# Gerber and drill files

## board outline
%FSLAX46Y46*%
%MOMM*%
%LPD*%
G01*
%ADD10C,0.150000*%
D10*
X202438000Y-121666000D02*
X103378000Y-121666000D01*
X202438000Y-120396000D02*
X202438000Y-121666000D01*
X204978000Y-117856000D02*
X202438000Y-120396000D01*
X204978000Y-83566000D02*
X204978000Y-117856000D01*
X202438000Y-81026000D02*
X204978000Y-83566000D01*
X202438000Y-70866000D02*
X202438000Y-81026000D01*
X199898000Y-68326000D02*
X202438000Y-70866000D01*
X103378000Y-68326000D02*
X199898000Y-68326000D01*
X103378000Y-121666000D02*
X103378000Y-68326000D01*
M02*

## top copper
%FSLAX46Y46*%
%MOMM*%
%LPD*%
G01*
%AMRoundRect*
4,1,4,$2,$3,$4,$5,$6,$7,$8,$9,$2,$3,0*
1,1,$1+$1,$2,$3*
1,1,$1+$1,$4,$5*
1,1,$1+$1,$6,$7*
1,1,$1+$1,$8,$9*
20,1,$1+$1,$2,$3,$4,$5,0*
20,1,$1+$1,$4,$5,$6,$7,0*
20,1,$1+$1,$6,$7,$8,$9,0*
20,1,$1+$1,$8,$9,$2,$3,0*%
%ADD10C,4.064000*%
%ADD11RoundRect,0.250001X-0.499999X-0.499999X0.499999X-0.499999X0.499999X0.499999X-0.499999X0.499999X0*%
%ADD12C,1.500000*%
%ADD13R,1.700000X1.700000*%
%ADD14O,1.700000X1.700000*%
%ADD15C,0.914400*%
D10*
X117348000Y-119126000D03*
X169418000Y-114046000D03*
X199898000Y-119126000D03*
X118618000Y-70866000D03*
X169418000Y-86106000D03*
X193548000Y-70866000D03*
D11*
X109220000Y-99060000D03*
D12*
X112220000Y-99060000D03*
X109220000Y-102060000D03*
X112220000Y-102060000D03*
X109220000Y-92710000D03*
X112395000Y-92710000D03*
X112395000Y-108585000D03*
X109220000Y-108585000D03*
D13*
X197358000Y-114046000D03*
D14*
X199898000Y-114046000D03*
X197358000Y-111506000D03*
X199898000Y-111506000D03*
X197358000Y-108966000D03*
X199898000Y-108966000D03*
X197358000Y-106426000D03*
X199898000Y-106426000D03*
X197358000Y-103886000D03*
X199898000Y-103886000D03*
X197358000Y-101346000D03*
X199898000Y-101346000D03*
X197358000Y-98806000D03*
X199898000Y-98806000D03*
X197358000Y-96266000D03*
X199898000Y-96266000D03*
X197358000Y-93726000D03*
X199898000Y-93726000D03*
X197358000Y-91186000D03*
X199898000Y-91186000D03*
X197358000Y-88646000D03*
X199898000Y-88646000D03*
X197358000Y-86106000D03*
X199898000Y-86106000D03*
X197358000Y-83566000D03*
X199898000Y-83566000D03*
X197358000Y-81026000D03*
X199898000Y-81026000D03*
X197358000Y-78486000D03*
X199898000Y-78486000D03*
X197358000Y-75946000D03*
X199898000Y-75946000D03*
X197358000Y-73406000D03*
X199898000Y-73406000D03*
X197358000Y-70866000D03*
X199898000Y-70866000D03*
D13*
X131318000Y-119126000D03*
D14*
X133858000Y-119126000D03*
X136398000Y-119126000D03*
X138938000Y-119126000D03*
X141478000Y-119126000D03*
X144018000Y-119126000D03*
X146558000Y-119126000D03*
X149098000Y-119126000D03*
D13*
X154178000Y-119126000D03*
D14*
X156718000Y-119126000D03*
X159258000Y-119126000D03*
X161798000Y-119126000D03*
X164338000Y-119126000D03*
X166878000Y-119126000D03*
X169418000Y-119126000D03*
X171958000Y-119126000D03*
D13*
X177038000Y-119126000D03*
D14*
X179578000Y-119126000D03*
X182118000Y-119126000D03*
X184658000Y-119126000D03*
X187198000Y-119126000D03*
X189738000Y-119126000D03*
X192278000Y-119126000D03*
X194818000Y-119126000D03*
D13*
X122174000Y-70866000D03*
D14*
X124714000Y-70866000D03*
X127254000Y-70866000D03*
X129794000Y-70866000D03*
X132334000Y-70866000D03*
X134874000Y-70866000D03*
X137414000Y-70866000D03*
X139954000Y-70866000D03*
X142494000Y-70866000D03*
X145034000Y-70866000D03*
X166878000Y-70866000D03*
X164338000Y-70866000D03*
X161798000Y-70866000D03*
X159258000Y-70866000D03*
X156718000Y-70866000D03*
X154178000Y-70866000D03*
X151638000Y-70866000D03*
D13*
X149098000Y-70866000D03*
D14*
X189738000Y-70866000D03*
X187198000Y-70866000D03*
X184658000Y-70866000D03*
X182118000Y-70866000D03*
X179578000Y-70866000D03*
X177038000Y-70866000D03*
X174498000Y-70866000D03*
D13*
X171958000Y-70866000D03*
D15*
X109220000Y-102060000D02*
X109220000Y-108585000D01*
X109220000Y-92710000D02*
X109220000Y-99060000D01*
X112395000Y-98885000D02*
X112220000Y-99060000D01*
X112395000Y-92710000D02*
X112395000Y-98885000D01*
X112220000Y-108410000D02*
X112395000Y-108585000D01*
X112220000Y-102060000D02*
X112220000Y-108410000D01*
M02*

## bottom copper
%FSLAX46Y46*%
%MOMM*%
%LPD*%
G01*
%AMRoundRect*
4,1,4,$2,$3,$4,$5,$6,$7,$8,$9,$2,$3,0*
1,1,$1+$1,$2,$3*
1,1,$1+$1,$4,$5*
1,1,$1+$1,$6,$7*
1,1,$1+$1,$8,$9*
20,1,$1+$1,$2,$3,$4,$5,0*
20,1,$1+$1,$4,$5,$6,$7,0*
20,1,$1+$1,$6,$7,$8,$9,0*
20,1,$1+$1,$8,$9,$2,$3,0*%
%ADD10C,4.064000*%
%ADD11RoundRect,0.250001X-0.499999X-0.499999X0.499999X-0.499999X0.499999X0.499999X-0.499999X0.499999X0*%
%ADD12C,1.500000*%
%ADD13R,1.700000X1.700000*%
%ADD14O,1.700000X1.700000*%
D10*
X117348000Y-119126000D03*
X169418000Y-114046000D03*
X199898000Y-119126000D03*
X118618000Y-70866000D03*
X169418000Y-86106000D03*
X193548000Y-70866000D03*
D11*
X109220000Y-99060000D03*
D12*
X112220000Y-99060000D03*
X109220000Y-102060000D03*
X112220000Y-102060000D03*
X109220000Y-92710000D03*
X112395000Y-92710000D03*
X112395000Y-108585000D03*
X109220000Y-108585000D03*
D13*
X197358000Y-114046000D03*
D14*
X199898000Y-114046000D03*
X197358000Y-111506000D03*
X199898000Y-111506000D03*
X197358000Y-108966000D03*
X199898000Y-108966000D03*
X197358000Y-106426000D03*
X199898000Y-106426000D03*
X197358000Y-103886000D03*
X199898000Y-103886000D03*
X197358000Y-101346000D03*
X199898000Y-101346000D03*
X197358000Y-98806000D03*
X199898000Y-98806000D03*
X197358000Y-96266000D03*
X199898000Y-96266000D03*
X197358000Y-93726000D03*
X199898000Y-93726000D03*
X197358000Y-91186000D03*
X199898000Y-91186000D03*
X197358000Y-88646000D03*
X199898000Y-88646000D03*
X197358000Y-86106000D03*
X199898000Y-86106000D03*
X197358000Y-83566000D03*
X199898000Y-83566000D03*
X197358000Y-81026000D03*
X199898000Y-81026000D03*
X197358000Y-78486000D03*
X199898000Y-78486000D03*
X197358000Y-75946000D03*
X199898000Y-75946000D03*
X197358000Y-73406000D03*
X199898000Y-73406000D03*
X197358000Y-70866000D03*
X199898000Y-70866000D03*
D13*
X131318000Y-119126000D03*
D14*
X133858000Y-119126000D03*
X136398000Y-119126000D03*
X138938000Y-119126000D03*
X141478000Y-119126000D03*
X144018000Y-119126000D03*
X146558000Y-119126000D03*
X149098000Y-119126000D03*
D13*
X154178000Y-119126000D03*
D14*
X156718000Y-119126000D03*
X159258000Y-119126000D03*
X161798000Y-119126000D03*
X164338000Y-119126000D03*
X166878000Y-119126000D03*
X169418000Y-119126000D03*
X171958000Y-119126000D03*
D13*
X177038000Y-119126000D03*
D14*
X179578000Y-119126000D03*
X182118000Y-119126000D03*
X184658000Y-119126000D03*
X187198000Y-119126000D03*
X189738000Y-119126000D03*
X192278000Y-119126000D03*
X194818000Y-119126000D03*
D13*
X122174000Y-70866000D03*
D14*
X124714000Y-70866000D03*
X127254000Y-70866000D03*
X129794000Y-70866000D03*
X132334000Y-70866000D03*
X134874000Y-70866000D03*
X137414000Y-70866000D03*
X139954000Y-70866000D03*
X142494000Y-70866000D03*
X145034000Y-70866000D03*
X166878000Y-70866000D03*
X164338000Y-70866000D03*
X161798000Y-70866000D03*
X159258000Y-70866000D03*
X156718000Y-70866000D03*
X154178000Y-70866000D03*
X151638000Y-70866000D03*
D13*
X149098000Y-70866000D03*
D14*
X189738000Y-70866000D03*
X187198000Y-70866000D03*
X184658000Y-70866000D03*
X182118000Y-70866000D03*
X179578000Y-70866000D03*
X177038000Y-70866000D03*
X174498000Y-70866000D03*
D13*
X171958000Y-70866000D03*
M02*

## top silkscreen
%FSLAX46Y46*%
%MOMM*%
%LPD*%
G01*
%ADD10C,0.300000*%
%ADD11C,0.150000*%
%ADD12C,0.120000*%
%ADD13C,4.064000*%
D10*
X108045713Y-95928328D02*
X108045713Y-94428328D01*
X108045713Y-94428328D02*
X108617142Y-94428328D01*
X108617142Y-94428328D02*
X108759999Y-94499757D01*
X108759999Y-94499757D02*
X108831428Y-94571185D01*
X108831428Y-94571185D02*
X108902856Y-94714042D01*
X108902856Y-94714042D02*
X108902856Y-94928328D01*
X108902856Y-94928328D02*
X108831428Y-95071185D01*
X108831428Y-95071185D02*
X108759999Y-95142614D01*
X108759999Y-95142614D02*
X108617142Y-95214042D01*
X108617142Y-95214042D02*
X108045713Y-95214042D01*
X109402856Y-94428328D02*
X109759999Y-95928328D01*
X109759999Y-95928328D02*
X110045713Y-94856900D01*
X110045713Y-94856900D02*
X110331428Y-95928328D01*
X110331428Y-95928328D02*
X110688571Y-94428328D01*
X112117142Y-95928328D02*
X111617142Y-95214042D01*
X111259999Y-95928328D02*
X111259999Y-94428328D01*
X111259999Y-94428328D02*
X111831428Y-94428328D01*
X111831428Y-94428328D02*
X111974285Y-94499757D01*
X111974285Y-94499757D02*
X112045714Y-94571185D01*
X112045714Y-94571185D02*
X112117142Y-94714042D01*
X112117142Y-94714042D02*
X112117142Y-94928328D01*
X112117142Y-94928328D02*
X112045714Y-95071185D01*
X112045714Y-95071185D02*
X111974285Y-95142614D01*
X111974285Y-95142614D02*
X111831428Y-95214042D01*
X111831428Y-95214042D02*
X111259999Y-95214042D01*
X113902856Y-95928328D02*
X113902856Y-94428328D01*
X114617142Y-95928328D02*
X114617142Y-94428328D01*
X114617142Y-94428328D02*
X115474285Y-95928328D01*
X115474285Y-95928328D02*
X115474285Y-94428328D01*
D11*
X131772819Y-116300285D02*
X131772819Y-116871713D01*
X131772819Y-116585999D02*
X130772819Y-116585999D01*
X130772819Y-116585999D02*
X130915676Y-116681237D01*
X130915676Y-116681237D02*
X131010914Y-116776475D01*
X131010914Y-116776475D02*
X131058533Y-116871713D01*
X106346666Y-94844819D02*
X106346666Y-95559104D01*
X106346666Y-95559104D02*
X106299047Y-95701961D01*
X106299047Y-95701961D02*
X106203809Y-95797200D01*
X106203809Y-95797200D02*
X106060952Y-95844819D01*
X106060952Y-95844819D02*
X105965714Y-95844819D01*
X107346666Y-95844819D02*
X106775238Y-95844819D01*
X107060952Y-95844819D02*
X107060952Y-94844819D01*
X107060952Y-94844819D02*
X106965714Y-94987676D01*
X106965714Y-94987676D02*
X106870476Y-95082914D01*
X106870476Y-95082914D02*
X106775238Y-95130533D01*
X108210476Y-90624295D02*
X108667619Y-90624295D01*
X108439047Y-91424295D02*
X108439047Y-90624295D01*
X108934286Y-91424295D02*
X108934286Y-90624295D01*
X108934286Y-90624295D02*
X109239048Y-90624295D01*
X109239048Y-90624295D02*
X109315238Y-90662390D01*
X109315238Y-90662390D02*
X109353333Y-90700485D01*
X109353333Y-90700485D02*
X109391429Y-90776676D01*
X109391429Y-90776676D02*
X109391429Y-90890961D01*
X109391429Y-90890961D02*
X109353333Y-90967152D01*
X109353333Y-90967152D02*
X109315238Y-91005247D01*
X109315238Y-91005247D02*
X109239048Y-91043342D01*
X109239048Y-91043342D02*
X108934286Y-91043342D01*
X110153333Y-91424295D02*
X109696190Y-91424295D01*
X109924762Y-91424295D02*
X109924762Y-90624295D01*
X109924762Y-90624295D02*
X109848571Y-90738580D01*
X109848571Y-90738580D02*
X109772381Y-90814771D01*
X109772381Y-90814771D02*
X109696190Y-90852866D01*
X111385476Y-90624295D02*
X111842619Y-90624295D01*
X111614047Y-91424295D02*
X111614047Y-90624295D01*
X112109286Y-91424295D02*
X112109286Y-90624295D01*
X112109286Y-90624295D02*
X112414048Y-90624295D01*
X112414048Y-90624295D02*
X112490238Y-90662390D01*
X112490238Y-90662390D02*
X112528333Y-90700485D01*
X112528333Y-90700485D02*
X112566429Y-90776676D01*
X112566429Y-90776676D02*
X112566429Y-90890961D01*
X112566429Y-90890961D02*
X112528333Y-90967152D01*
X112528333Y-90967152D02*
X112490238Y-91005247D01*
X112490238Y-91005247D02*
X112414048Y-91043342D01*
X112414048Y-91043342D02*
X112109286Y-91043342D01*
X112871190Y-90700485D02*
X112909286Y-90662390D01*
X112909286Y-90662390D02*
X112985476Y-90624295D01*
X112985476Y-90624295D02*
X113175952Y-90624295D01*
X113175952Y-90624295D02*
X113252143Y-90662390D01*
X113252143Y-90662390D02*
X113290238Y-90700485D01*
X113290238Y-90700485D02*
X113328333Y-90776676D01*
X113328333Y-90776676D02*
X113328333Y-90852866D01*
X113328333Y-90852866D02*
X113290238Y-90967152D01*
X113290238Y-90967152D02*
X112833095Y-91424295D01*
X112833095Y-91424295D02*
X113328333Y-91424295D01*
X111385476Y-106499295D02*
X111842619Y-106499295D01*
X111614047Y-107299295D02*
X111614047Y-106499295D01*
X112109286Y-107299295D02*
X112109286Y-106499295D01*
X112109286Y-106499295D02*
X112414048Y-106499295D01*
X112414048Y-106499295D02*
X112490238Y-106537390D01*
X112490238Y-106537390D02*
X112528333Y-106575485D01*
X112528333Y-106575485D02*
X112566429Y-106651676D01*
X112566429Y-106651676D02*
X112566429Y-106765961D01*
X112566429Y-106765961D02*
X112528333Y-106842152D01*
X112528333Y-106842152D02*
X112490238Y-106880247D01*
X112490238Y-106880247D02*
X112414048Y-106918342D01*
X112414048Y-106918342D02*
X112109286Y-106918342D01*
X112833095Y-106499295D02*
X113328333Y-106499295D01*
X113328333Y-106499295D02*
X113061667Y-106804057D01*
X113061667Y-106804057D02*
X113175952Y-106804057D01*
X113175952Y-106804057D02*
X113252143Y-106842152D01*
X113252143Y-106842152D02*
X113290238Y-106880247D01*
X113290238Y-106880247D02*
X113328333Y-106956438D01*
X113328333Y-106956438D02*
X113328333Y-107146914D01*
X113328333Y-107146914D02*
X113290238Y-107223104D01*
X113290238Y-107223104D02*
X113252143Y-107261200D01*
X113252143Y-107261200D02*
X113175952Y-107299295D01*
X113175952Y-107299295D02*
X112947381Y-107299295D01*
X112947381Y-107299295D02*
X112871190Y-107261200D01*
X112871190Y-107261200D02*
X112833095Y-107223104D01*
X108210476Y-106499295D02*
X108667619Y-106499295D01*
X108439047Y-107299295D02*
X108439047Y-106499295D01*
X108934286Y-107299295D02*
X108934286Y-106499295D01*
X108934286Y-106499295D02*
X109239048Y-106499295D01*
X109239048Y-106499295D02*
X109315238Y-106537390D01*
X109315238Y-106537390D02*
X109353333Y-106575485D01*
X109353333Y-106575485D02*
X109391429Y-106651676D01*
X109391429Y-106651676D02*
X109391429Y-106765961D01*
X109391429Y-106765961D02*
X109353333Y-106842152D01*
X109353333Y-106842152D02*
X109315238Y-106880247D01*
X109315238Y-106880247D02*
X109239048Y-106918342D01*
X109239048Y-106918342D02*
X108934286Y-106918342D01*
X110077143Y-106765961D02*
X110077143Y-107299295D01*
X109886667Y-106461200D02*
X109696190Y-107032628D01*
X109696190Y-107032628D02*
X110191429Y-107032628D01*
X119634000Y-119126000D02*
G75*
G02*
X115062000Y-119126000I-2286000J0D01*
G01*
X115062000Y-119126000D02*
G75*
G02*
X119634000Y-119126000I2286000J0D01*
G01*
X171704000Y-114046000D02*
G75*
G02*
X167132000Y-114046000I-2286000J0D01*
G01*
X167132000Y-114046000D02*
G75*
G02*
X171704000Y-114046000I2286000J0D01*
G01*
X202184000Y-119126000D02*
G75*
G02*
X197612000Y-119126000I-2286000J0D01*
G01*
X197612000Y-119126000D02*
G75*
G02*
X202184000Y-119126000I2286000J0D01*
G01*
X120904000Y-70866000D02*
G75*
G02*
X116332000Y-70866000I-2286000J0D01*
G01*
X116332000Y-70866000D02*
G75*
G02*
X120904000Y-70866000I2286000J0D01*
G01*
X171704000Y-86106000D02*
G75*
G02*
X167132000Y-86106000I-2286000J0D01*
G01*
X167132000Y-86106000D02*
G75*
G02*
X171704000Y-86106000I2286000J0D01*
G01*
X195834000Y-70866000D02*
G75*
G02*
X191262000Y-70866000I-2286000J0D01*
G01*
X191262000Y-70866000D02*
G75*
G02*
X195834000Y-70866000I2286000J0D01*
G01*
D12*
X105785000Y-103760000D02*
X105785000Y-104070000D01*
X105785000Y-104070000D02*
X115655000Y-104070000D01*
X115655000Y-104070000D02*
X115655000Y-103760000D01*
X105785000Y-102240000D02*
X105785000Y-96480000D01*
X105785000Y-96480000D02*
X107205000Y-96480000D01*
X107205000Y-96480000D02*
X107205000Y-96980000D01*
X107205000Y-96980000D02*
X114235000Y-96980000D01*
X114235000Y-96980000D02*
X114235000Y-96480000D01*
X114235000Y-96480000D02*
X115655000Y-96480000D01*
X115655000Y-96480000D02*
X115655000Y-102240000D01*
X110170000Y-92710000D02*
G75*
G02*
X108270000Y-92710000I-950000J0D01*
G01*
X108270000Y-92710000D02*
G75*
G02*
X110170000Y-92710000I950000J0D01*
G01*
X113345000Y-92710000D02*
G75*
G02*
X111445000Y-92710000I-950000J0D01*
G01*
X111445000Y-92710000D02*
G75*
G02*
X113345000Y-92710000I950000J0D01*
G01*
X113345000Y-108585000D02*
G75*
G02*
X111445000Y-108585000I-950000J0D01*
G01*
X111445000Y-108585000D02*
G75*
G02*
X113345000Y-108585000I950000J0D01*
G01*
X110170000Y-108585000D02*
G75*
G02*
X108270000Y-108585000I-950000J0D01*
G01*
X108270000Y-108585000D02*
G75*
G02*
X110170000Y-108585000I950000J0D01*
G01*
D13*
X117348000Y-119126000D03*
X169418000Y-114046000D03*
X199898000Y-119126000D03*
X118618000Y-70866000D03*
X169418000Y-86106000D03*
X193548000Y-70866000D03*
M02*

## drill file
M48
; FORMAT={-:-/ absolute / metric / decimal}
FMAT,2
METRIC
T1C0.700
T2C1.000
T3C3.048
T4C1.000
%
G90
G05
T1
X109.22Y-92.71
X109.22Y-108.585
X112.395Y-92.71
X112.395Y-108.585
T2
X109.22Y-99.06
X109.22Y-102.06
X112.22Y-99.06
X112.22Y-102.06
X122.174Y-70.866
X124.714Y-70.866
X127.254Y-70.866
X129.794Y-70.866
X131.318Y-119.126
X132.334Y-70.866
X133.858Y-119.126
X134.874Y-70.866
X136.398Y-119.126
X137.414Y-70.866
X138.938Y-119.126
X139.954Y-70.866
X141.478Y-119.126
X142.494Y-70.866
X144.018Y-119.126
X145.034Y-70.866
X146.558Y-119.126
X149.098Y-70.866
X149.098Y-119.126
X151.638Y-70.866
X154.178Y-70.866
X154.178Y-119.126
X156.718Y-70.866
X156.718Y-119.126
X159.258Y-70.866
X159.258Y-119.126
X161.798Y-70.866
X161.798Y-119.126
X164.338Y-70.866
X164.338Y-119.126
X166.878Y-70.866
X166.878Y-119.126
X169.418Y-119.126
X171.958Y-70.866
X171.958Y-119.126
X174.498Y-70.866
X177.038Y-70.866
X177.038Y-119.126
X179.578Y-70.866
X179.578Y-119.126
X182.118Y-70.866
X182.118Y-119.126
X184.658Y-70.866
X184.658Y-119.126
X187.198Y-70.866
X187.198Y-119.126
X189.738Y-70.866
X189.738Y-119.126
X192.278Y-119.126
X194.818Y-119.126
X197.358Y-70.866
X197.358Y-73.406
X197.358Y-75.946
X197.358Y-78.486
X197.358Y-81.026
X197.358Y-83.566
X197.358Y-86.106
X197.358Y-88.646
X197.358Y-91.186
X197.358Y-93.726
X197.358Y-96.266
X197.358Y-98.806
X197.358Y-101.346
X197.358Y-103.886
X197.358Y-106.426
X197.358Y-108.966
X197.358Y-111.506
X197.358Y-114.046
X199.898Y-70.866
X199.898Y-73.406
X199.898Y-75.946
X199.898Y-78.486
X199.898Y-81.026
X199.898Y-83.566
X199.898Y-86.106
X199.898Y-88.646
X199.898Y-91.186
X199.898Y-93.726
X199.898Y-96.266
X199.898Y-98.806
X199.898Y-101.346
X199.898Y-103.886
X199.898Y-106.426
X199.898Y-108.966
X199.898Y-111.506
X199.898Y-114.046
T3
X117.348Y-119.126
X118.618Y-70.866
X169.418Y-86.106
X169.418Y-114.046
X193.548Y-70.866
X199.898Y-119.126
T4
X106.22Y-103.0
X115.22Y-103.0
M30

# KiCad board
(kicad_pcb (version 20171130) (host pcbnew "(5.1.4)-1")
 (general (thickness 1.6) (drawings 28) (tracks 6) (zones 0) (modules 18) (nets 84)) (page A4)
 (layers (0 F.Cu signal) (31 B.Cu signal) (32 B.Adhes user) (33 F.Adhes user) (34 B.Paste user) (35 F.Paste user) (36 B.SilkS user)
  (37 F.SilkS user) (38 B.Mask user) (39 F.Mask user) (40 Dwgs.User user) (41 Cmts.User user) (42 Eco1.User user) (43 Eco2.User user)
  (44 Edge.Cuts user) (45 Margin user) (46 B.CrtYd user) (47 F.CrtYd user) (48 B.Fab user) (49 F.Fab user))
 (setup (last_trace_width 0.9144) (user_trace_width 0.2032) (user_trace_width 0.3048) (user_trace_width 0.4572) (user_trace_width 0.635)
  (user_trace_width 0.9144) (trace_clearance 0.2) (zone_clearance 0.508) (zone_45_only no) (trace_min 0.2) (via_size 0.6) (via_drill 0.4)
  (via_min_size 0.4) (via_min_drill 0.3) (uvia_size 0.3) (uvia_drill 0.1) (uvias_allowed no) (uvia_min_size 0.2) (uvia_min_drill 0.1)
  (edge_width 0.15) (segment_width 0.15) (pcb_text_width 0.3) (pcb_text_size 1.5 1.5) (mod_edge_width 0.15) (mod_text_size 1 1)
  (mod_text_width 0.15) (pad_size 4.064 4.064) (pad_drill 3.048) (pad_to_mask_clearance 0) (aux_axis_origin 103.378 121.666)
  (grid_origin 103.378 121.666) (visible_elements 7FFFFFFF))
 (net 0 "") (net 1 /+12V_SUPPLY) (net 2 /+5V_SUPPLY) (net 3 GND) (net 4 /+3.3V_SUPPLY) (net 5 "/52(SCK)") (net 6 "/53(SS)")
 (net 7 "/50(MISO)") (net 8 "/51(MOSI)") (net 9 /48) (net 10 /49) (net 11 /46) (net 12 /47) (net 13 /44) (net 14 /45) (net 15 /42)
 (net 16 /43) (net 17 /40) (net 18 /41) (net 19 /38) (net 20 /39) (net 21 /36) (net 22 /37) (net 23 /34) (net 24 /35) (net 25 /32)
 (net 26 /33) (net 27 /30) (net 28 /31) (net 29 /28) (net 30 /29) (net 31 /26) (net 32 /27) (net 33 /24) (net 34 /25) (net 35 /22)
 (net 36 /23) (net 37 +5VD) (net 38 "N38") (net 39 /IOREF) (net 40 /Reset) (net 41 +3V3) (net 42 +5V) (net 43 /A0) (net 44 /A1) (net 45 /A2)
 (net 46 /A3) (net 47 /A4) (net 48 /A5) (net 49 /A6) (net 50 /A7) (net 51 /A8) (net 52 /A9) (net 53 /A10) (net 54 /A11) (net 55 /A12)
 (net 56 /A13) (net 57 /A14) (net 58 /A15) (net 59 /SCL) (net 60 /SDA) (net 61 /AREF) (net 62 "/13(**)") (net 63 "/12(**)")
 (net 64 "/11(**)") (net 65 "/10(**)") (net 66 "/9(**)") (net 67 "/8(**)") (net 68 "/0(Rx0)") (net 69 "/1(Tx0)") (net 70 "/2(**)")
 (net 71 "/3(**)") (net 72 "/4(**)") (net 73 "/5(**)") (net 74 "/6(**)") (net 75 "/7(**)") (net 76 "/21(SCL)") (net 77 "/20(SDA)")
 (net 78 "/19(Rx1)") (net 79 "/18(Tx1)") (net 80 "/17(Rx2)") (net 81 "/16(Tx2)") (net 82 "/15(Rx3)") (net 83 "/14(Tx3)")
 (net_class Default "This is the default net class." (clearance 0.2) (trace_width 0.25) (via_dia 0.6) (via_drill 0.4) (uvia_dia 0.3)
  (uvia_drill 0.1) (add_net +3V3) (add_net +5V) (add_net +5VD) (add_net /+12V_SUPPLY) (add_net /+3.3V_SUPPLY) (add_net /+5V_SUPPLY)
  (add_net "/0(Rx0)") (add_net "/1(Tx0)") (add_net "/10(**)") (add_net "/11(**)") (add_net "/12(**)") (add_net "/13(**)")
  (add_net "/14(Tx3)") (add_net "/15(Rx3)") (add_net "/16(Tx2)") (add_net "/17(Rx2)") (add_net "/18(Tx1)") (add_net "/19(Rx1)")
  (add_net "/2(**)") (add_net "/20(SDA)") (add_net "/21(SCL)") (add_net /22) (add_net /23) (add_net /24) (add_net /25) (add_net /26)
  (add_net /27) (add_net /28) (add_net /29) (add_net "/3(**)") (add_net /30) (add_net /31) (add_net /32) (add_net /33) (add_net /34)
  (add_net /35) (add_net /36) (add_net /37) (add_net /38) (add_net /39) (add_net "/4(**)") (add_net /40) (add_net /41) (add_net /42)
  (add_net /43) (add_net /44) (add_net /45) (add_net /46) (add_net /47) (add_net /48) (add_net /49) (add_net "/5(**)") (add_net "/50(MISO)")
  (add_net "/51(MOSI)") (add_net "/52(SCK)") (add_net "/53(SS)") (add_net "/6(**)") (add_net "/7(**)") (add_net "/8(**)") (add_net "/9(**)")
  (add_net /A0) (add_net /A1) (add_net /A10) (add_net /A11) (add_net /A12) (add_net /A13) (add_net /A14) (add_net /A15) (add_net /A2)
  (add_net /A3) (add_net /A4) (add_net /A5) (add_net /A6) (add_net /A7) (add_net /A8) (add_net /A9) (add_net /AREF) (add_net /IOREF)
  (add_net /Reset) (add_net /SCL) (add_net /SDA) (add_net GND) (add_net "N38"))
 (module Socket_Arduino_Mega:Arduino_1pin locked (layer F.Cu) (at 117.348 119.126)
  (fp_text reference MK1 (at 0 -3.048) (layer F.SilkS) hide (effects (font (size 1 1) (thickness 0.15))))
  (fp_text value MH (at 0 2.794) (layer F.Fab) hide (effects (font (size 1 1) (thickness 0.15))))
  (fp_circle (center 0 0) (end 0 -2.286) (layer F.SilkS) (width 0.15))
  (pad 1 thru_hole circle (at 0 0) (size 4.064 4.064) (drill 3.048) (layers *.Cu *.Mask F.SilkS)))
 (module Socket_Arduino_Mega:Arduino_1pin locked (layer F.Cu) (at 169.418 114.046)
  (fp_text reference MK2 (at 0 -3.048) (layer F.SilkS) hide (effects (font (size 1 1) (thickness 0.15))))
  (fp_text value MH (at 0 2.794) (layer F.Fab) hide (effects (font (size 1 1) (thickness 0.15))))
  (fp_circle (center 0 0) (end 0 -2.286) (layer F.SilkS) (width 0.15))
  (pad 1 thru_hole circle (at 0 0) (size 4.064 4.064) (drill 3.048) (layers *.Cu *.Mask F.SilkS)))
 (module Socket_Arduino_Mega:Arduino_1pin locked (layer F.Cu) (at 199.898 119.126)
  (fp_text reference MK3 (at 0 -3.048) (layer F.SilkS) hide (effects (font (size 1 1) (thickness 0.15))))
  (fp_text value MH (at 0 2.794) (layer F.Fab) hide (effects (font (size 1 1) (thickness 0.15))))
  (fp_circle (center 0 0) (end 0 -2.286) (layer F.SilkS) (width 0.15))
  (pad 1 thru_hole circle (at 0 0) (size 4.064 4.064) (drill 3.048) (layers *.Cu *.Mask F.SilkS)))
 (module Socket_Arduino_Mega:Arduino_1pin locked (layer F.Cu) (at 118.618 70.866)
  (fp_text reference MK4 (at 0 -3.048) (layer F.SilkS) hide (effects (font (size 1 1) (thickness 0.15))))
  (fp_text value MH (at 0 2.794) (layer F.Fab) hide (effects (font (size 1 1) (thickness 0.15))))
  (fp_circle (center 0 0) (end 0 -2.286) (layer F.SilkS) (width 0.15))
  (pad 1 thru_hole circle (at 0 0) (size 4.064 4.064) (drill 3.048) (layers *.Cu *.Mask F.SilkS)))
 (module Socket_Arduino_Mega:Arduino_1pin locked (layer F.Cu) (at 169.418 86.106)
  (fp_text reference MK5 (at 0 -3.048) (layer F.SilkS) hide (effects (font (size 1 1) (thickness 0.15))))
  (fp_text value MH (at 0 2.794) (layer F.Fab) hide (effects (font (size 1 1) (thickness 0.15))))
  (fp_circle (center 0 0) (end 0 -2.286) (layer F.SilkS) (width 0.15))
  (pad 1 thru_hole circle (at 0 0) (size 4.064 4.064) (drill 3.048) (layers *.Cu *.Mask F.SilkS)))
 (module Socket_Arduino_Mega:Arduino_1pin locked (layer F.Cu) (at 193.548 70.866)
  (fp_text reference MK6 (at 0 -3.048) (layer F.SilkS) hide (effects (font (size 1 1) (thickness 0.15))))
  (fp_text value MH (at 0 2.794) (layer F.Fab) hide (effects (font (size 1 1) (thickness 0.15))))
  (fp_circle (center 0 0) (end 0 -2.286) (layer F.SilkS) (width 0.15))
  (pad 1 thru_hole circle (at 0 0) (size 4.064 4.064) (drill 3.048) (layers *.Cu *.Mask F.SilkS)))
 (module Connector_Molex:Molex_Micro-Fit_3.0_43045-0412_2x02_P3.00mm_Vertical (layer F.Cu) (at 109.22 99.06)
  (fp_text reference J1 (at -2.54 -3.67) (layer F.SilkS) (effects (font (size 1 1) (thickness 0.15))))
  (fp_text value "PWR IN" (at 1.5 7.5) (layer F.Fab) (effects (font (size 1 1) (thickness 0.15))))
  (fp_line (start -3.435 4.7) (end -3.435 5.01) (layer F.SilkS) (width 0.12))
  (fp_line (start -3.435 5.01) (end 6.435 5.01) (layer F.SilkS) (width 0.12))
  (fp_line (start 6.435 5.01) (end 6.435 4.7) (layer F.SilkS) (width 0.12))
  (fp_line (start -3.435 3.18) (end -3.435 -2.58) (layer F.SilkS) (width 0.12))
  (fp_line (start -3.435 -2.58) (end -2.015 -2.58) (layer F.SilkS) (width 0.12))
  (fp_line (start -2.015 -2.58) (end -2.015 -2.08) (layer F.SilkS) (width 0.12))
  (fp_line (start -2.015 -2.08) (end 5.015 -2.08) (layer F.SilkS) (width 0.12))
  (fp_line (start 5.015 -2.08) (end 5.015 -2.58) (layer F.SilkS) (width 0.12))
  (fp_line (start 5.015 -2.58) (end 6.435 -2.58) (layer F.SilkS) (width 0.12))
  (fp_line (start 6.435 -2.58) (end 6.435 3.18) (layer F.SilkS) (width 0.12))
  (pad "" np_thru_hole circle (at -3 3.94) (size 1 1) (drill 1) (layers *.Cu *.Mask))
  (pad "" np_thru_hole circle (at 6 3.94) (size 1 1) (drill 1) (layers *.Cu *.Mask))
  (pad 1 thru_hole roundrect (at 0 0) (size 1.5 1.5) (drill 1) (layers *.Cu *.Mask) (roundrect_rratio 0.166667) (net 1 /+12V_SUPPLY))
  (pad 2 thru_hole circle (at 3 0) (size 1.5 1.5) (drill 1) (layers *.Cu *.Mask) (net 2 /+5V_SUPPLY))
  (pad 3 thru_hole circle (at 0 3) (size 1.5 1.5) (drill 1) (layers *.Cu *.Mask) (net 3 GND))
  (pad 4 thru_hole circle (at 3 3) (size 1.5 1.5) (drill 1) (layers *.Cu *.Mask) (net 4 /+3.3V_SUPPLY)))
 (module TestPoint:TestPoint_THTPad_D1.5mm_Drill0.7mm (layer F.Cu) (at 109.22 92.71)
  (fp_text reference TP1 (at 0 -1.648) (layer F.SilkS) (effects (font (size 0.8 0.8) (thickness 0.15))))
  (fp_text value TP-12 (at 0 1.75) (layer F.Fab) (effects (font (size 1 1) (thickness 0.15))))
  (fp_circle (center 0 0) (end 0 0.95) (layer F.SilkS) (width 0.12))
  (pad 1 thru_hole circle (at 0 0) (size 1.5 1.5) (drill 0.7) (layers *.Cu *.Mask) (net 1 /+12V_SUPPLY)))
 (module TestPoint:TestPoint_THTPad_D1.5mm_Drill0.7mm (layer F.Cu) (at 112.395 92.71)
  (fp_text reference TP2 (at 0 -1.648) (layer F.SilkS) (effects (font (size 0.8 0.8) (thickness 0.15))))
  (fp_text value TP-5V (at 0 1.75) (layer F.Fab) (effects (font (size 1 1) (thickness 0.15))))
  (fp_circle (center 0 0) (end 0 0.95) (layer F.SilkS) (width 0.12))
  (pad 1 thru_hole circle (at 0 0) (size 1.5 1.5) (drill 0.7) (layers *.Cu *.Mask) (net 2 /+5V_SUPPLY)))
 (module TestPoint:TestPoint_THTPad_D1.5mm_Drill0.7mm (layer F.Cu) (at 112.395 108.585)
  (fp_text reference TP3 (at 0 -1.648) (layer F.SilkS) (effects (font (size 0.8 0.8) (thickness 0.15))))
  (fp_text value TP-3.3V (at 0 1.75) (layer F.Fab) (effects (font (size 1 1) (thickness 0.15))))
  (fp_circle (center 0 0) (end 0 0.95) (layer F.SilkS) (width 0.12))
  (pad 1 thru_hole circle (at 0 0) (size 1.5 1.5) (drill 0.7) (layers *.Cu *.Mask) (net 4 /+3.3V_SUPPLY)))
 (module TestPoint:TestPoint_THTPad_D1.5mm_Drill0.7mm (layer F.Cu) (at 109.22 108.585)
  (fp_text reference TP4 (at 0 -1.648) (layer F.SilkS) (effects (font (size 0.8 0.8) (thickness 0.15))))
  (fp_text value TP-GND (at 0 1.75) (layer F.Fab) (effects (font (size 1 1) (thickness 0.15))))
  (fp_circle (center 0 0) (end 0 0.95) (layer F.SilkS) (width 0.12))
  (pad 1 thru_hole circle (at 0 0) (size 1.5 1.5) (drill 0.7) (layers *.Cu *.Mask) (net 3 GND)))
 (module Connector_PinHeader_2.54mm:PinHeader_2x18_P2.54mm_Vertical (layer B.Cu) (at 197.358 114.046)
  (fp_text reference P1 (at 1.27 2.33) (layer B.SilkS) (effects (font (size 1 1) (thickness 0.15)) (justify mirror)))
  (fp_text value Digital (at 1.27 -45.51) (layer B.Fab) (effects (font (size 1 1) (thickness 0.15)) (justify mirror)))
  (pad 1 thru_hole rect (at 0 0) (size 1.7 1.7) (drill 1) (layers *.Cu *.Mask) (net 3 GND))
  (pad 2 thru_hole oval (at 2.54 0) (size 1.7 1.7) (drill 1) (layers *.Cu *.Mask) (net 3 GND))
  (pad 3 thru_hole oval (at 0 -2.54) (size 1.7 1.7) (drill 1) (layers *.Cu *.Mask) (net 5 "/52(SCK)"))
  (pad 4 thru_hole oval (at 2.54 -2.54) (size 1.7 1.7) (drill 1) (layers *.Cu *.Mask) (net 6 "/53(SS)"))
  (pad 5 thru_hole oval (at 0 -5.08) (size 1.7 1.7) (drill 1) (layers *.Cu *.Mask) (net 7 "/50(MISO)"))
  (pad 6 thru_hole oval (at 2.54 -5.08) (size 1.7 1.7) (drill 1) (layers *.Cu *.Mask) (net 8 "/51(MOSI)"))
  (pad 7 thru_hole oval (at 0 -7.62) (size 1.7 1.7) (drill 1) (layers *.Cu *.Mask) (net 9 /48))
  (pad 8 thru_hole oval (at 2.54 -7.62) (size 1.7 1.7) (drill 1) (layers *.Cu *.Mask) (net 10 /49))
  (pad 9 thru_hole oval (at 0 -10.16) (size 1.7 1.7) (drill 1) (layers *.Cu *.Mask) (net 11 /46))
  (pad 10 thru_hole oval (at 2.54 -10.16) (size 1.7 1.7) (drill 1) (layers *.Cu *.Mask) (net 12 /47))
  (pad 11 thru_hole oval (at 0 -12.7) (size 1.7 1.7) (drill 1) (layers *.Cu *.Mask) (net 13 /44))
  (pad 12 thru_hole oval (at 2.54 -12.7) (size 1.7 1.7) (drill 1) (layers *.Cu *.Mask) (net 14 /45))
  (pad 13 thru_hole oval (at 0 -15.24) (size 1.7 1.7) (drill 1) (layers *.Cu *.Mask) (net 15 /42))
  (pad 14 thru_hole oval (at 2.54 -15.24) (size 1.7 1.7) (drill 1) (layers *.Cu *.Mask) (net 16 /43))
  (pad 15 thru_hole oval (at 0 -17.78) (size 1.7 1.7) (drill 1) (layers *.Cu *.Mask) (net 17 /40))
  (pad 16 thru_hole oval (at 2.54 -17.78) (size 1.7 1.7) (drill 1) (layers *.Cu *.Mask) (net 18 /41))
  (pad 17 thru_hole oval (at 0 -20.32) (size 1.7 1.7) (drill 1) (layers *.Cu *.Mask) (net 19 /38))
  (pad 18 thru_hole oval (at 2.54 -20.32) (size 1.7 1.7) (drill 1) (layers *.Cu *.Mask) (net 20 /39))
  (pad 19 thru_hole oval (at 0 -22.86) (size 1.7 1.7) (drill 1) (layers *.Cu *.Mask) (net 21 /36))
  (pad 20 thru_hole oval (at 2.54 -22.86) (size 1.7 1.7) (drill 1) (layers *.Cu *.Mask) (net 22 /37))
  (pad 21 thru_hole oval (at 0 -25.4) (size 1.7 1.7) (drill 1) (layers *.Cu *.Mask) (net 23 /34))
  (pad 22 thru_hole oval (at 2.54 -25.4) (size 1.7 1.7) (drill 1) (layers *.Cu *.Mask) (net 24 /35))
  (pad 23 thru_hole oval (at 0 -27.94) (size 1.7 1.7) (drill 1) (layers *.Cu *.Mask) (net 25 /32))
  (pad 24 thru_hole oval (at 2.54 -27.94) (size 1.7 1.7) (drill 1) (layers *.Cu *.Mask) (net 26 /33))
  (pad 25 thru_hole oval (at 0 -30.48) (size 1.7 1.7) (drill 1) (layers *.Cu *.Mask) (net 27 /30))
  (pad 26 thru_hole oval (at 2.54 -30.48) (size 1.7 1.7) (drill 1) (layers *.Cu *.Mask) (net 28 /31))
  (pad 27 thru_hole oval (at 0 -33.02) (size 1.7 1.7) (drill 1) (layers *.Cu *.Mask) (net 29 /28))
  (pad 28 thru_hole oval (at 2.54 -33.02) (size 1.7 1.7) (drill 1) (layers *.Cu *.Mask) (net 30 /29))
  (pad 29 thru_hole oval (at 0 -35.56) (size 1.7 1.7) (drill 1) (layers *.Cu *.Mask) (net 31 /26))
  (pad 30 thru_hole oval (at 2.54 -35.56) (size 1.7 1.7) (drill 1) (layers *.Cu *.Mask) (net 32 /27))
  (pad 31 thru_hole oval (at 0 -38.1) (size 1.7 1.7) (drill 1) (layers *.Cu *.Mask) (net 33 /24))
  (pad 32 thru_hole oval (at 2.54 -38.1) (size 1.7 1.7) (drill 1) (layers *.Cu *.Mask) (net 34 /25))
  (pad 33 thru_hole oval (at 0 -40.64) (size 1.7 1.7) (drill 1) (layers *.Cu *.Mask) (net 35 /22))
  (pad 34 thru_hole oval (at 2.54 -40.64) (size 1.7 1.7) (drill 1) (layers *.Cu *.Mask) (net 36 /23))
  (pad 35 thru_hole oval (at 0 -43.18) (size 1.7 1.7) (drill 1) (layers *.Cu *.Mask) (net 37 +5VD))
  (pad 36 thru_hole oval (at 2.54 -43.18) (size 1.7 1.7) (drill 1) (layers *.Cu *.Mask) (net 37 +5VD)))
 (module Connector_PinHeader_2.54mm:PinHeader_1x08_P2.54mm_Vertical (layer B.Cu) (at 131.318 119.126 270)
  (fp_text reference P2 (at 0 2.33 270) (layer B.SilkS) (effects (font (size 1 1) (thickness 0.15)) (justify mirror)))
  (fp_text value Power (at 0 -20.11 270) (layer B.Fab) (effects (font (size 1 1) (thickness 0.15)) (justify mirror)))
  (pad 1 thru_hole rect (at 0 0 270) (size 1.7 1.7) (drill 1) (layers *.Cu *.Mask) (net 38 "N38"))
  (pad 2 thru_hole oval (at 0 -2.54 270) (size 1.7 1.7) (drill 1) (layers *.Cu *.Mask) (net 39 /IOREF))
  (pad 3 thru_hole oval (at 0 -5.08 270) (size 1.7 1.7) (drill 1) (layers *.Cu *.Mask) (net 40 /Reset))
  (pad 4 thru_hole oval (at 0 -7.62 270) (size 1.7 1.7) (drill 1) (layers *.Cu *.Mask) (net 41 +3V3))
  (pad 5 thru_hole oval (at 0 -10.16 270) (size 1.7 1.7) (drill 1) (layers *.Cu *.Mask) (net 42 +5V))
  (pad 6 thru_hole oval (at 0 -12.7 270) (size 1.7 1.7) (drill 1) (layers *.Cu *.Mask) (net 3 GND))
  (pad 7 thru_hole oval (at 0 -15.24 270) (size 1.7 1.7) (drill 1) (layers *.Cu *.Mask) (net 3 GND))
  (pad 8 thru_hole oval (at 0 -17.78 270) (size 1.7 1.7) (drill 1) (layers *.Cu *.Mask) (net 1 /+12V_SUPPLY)))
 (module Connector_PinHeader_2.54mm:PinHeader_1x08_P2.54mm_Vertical (layer B.Cu) (at 154.178 119.126 270)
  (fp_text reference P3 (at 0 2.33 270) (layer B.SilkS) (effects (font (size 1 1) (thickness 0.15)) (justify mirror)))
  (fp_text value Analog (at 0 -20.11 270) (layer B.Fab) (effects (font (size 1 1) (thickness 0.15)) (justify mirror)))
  (pad 1 thru_hole rect (at 0 0 270) (size 1.7 1.7) (drill 1) (layers *.Cu *.Mask) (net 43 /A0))
  (pad 2 thru_hole oval (at 0 -2.54 270) (size 1.7 1.7) (drill 1) (layers *.Cu *.Mask) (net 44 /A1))
  (pad 3 thru_hole oval (at 0 -5.08 270) (size 1.7 1.7) (drill 1) (layers *.Cu *.Mask) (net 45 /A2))
  (pad 4 thru_hole oval (at 0 -7.62 270) (size 1.7 1.7) (drill 1) (layers *.Cu *.Mask) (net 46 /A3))
  (pad 5 thru_hole oval (at 0 -10.16 270) (size 1.7 1.7) (drill 1) (layers *.Cu *.Mask) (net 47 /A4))
  (pad 6 thru_hole oval (at 0 -12.7 270) (size 1.7 1.7) (drill 1) (layers *.Cu *.Mask) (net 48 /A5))
  (pad 7 thru_hole oval (at 0 -15.24 270) (size 1.7 1.7) (drill 1) (layers *.Cu *.Mask) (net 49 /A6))
  (pad 8 thru_hole oval (at 0 -17.78 270) (size 1.7 1.7) (drill 1) (layers *.Cu *.Mask) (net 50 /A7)))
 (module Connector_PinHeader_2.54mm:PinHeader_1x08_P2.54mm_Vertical (layer B.Cu) (at 177.038 119.126 270)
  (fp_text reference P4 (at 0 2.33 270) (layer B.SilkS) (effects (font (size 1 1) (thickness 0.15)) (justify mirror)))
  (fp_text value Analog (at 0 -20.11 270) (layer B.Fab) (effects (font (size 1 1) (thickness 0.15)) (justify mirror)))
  (pad 1 thru_hole rect (at 0 0 270) (size 1.7 1.7) (drill 1) (layers *.Cu *.Mask) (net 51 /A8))
  (pad 2 thru_hole oval (at 0 -2.54 270) (size 1.7 1.7) (drill 1) (layers *.Cu *.Mask) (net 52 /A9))
  (pad 3 thru_hole oval (at 0 -5.08 270) (size 1.7 1.7) (drill 1) (layers *.Cu *.Mask) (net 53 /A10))
  (pad 4 thru_hole oval (at 0 -7.62 270) (size 1.7 1.7) (drill 1) (layers *.Cu *.Mask) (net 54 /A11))
  (pad 5 thru_hole oval (at 0 -10.16 270) (size 1.7 1.7) (drill 1) (layers *.Cu *.Mask) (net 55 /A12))
  (pad 6 thru_hole oval (at 0 -12.7 270) (size 1.7 1.7) (drill 1) (layers *.Cu *.Mask) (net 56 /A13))
  (pad 7 thru_hole oval (at 0 -15.24 270) (size 1.7 1.7) (drill 1) (layers *.Cu *.Mask) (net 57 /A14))
  (pad 8 thru_hole oval (at 0 -17.78 270) (size 1.7 1.7) (drill 1) (layers *.Cu *.Mask) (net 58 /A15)))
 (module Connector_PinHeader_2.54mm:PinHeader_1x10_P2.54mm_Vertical (layer B.Cu) (at 122.174 70.866 270)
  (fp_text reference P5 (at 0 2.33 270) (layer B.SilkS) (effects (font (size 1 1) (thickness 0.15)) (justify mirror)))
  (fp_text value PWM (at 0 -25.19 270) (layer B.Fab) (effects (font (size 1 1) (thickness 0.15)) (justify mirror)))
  (pad 1 thru_hole rect (at 0 0 270) (size 1.7 1.7) (drill 1) (layers *.Cu *.Mask) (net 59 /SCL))
  (pad 2 thru_hole oval (at 0 -2.54 270) (size 1.7 1.7) (drill 1) (layers *.Cu *.Mask) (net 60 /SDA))
  (pad 3 thru_hole oval (at 0 -5.08 270) (size 1.7 1.7) (drill 1) (layers *.Cu *.Mask) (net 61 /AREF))
  (pad 4 thru_hole oval (at 0 -7.62 270) (size 1.7 1.7) (drill 1) (layers *.Cu *.Mask) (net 3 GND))
  (pad 5 thru_hole oval (at 0 -10.16 270) (size 1.7 1.7) (drill 1) (layers *.Cu *.Mask) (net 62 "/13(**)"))
  (pad 6 thru_hole oval (at 0 -12.7 270) (size 1.7 1.7) (drill 1) (layers *.Cu *.Mask) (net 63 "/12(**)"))
  (pad 7 thru_hole oval (at 0 -15.24 270) (size 1.7 1.7) (drill 1) (layers *.Cu *.Mask) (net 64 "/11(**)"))
  (pad 8 thru_hole oval (at 0 -17.78 270) (size 1.7 1.7) (drill 1) (layers *.Cu *.Mask) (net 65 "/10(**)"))
  (pad 9 thru_hole oval (at 0 -20.32 270) (size 1.7 1.7) (drill 1) (layers *.Cu *.Mask) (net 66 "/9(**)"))
  (pad 10 thru_hole oval (at 0 -22.86 270) (size 1.7 1.7) (drill 1) (layers *.Cu *.Mask) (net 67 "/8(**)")))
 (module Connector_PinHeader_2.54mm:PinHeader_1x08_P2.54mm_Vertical (layer B.Cu) (at 149.098 70.866 270)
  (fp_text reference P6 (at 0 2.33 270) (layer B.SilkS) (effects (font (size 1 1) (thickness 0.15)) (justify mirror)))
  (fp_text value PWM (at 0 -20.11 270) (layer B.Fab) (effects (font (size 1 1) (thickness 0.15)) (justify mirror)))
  (pad 8 thru_hole oval (at 0 -17.78 270) (size 1.7 1.7) (drill 1) (layers *.Cu *.Mask) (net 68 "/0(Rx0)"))
  (pad 7 thru_hole oval (at 0 -15.24 270) (size 1.7 1.7) (drill 1) (layers *.Cu *.Mask) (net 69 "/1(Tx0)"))
  (pad 6 thru_hole oval (at 0 -12.7 270) (size 1.7 1.7) (drill 1) (layers *.Cu *.Mask) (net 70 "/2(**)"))
  (pad 5 thru_hole oval (at 0 -10.16 270) (size 1.7 1.7) (drill 1) (layers *.Cu *.Mask) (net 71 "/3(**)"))
  (pad 4 thru_hole oval (at 0 -7.62 270) (size 1.7 1.7) (drill 1) (layers *.Cu *.Mask) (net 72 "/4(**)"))
  (pad 3 thru_hole oval (at 0 -5.08 270) (size 1.7 1.7) (drill 1) (layers *.Cu *.Mask) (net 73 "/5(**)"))
  (pad 2 thru_hole oval (at 0 -2.54 270) (size 1.7 1.7) (drill 1) (layers *.Cu *.Mask) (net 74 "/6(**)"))
  (pad 1 thru_hole rect (at 0 0 270) (size 1.7 1.7) (drill 1) (layers *.Cu *.Mask) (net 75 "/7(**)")))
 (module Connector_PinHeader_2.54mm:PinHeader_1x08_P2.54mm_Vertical (layer B.Cu) (at 171.958 70.866 270)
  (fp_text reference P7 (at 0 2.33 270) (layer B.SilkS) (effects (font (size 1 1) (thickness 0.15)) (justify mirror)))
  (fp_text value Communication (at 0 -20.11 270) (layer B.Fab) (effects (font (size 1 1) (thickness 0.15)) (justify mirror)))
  (pad 8 thru_hole oval (at 0 -17.78 270) (size 1.7 1.7) (drill 1) (layers *.Cu *.Mask) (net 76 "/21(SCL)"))
  (pad 7 thru_hole oval (at 0 -15.24 270) (size 1.7 1.7) (drill 1) (layers *.Cu *.Mask) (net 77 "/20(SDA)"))
  (pad 6 thru_hole oval (at 0 -12.7 270) (size 1.7 1.7) (drill 1) (layers *.Cu *.Mask) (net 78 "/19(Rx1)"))
  (pad 5 thru_hole oval (at 0 -10.16 270) (size 1.7 1.7) (drill 1) (layers *.Cu *.Mask) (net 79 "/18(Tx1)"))
  (pad 4 thru_hole oval (at 0 -7.62 270) (size 1.7 1.7) (drill 1) (layers *.Cu *.Mask) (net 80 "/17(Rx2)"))
  (pad 3 thru_hole oval (at 0 -5.08 270) (size 1.7 1.7) (drill 1) (layers *.Cu *.Mask) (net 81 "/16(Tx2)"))
  (pad 2 thru_hole oval (at 0 -2.54 270) (size 1.7 1.7) (drill 1) (layers *.Cu *.Mask) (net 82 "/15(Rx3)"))
  (pad 1 thru_hole rect (at 0 0 270) (size 1.7 1.7) (drill 1) (layers *.Cu *.Mask) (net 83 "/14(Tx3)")))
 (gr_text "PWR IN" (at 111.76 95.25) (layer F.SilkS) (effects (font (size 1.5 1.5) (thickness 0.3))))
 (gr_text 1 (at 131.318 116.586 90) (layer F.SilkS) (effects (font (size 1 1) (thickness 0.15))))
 (gr_line (start 202.438 121.666) (end 103.378 121.666) (angle 90) (layer Edge.Cuts) (width 0.15))
 (gr_line (start 202.438 120.396) (end 202.438 121.666) (angle 90) (layer Edge.Cuts) (width 0.15))
 (gr_line (start 204.978 117.856) (end 202.438 120.396) (angle 90) (layer Edge.Cuts) (width 0.15))
 (gr_line (start 204.978 83.566) (end 204.978 117.856) (angle 90) (layer Edge.Cuts) (width 0.15))
 (gr_line (start 202.438 81.026) (end 204.978 83.566) (angle 90) (layer Edge.Cuts) (width 0.15))
 (gr_line (start 202.438 70.866) (end 202.438 81.026) (angle 90) (layer Edge.Cuts) (width 0.15))
 (gr_line (start 199.898 68.326) (end 202.438 70.866) (angle 90) (layer Edge.Cuts) (width 0.15))
 (gr_line (start 103.378 68.326) (end 199.898 68.326) (angle 90) (layer Edge.Cuts) (width 0.15))
 (gr_line (start 103.378 121.666) (end 103.378 68.326) (angle 90) (layer Edge.Cuts) (width 0.15))
 (segment (start 109.22 102.06) (end 109.22 108.585) (width 0.9144) (layer F.Cu) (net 3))
 (segment (start 109.22 92.71) (end 109.22 99.06) (width 0.9144) (layer F.Cu) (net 1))
 (segment (start 112.395 98.885) (end 112.22 99.06) (width 0.9144) (layer F.Cu) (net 2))
 (segment (start 112.395 92.71) (end 112.395 98.885) (width 0.9144) (layer F.Cu) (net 2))
 (segment (start 112.22 108.41) (end 112.395 108.585) (width 0.9144) (layer F.Cu) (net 4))
 (segment (start 112.22 102.06) (end 112.22 108.41) (width 0.9144) (layer F.Cu) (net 4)))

